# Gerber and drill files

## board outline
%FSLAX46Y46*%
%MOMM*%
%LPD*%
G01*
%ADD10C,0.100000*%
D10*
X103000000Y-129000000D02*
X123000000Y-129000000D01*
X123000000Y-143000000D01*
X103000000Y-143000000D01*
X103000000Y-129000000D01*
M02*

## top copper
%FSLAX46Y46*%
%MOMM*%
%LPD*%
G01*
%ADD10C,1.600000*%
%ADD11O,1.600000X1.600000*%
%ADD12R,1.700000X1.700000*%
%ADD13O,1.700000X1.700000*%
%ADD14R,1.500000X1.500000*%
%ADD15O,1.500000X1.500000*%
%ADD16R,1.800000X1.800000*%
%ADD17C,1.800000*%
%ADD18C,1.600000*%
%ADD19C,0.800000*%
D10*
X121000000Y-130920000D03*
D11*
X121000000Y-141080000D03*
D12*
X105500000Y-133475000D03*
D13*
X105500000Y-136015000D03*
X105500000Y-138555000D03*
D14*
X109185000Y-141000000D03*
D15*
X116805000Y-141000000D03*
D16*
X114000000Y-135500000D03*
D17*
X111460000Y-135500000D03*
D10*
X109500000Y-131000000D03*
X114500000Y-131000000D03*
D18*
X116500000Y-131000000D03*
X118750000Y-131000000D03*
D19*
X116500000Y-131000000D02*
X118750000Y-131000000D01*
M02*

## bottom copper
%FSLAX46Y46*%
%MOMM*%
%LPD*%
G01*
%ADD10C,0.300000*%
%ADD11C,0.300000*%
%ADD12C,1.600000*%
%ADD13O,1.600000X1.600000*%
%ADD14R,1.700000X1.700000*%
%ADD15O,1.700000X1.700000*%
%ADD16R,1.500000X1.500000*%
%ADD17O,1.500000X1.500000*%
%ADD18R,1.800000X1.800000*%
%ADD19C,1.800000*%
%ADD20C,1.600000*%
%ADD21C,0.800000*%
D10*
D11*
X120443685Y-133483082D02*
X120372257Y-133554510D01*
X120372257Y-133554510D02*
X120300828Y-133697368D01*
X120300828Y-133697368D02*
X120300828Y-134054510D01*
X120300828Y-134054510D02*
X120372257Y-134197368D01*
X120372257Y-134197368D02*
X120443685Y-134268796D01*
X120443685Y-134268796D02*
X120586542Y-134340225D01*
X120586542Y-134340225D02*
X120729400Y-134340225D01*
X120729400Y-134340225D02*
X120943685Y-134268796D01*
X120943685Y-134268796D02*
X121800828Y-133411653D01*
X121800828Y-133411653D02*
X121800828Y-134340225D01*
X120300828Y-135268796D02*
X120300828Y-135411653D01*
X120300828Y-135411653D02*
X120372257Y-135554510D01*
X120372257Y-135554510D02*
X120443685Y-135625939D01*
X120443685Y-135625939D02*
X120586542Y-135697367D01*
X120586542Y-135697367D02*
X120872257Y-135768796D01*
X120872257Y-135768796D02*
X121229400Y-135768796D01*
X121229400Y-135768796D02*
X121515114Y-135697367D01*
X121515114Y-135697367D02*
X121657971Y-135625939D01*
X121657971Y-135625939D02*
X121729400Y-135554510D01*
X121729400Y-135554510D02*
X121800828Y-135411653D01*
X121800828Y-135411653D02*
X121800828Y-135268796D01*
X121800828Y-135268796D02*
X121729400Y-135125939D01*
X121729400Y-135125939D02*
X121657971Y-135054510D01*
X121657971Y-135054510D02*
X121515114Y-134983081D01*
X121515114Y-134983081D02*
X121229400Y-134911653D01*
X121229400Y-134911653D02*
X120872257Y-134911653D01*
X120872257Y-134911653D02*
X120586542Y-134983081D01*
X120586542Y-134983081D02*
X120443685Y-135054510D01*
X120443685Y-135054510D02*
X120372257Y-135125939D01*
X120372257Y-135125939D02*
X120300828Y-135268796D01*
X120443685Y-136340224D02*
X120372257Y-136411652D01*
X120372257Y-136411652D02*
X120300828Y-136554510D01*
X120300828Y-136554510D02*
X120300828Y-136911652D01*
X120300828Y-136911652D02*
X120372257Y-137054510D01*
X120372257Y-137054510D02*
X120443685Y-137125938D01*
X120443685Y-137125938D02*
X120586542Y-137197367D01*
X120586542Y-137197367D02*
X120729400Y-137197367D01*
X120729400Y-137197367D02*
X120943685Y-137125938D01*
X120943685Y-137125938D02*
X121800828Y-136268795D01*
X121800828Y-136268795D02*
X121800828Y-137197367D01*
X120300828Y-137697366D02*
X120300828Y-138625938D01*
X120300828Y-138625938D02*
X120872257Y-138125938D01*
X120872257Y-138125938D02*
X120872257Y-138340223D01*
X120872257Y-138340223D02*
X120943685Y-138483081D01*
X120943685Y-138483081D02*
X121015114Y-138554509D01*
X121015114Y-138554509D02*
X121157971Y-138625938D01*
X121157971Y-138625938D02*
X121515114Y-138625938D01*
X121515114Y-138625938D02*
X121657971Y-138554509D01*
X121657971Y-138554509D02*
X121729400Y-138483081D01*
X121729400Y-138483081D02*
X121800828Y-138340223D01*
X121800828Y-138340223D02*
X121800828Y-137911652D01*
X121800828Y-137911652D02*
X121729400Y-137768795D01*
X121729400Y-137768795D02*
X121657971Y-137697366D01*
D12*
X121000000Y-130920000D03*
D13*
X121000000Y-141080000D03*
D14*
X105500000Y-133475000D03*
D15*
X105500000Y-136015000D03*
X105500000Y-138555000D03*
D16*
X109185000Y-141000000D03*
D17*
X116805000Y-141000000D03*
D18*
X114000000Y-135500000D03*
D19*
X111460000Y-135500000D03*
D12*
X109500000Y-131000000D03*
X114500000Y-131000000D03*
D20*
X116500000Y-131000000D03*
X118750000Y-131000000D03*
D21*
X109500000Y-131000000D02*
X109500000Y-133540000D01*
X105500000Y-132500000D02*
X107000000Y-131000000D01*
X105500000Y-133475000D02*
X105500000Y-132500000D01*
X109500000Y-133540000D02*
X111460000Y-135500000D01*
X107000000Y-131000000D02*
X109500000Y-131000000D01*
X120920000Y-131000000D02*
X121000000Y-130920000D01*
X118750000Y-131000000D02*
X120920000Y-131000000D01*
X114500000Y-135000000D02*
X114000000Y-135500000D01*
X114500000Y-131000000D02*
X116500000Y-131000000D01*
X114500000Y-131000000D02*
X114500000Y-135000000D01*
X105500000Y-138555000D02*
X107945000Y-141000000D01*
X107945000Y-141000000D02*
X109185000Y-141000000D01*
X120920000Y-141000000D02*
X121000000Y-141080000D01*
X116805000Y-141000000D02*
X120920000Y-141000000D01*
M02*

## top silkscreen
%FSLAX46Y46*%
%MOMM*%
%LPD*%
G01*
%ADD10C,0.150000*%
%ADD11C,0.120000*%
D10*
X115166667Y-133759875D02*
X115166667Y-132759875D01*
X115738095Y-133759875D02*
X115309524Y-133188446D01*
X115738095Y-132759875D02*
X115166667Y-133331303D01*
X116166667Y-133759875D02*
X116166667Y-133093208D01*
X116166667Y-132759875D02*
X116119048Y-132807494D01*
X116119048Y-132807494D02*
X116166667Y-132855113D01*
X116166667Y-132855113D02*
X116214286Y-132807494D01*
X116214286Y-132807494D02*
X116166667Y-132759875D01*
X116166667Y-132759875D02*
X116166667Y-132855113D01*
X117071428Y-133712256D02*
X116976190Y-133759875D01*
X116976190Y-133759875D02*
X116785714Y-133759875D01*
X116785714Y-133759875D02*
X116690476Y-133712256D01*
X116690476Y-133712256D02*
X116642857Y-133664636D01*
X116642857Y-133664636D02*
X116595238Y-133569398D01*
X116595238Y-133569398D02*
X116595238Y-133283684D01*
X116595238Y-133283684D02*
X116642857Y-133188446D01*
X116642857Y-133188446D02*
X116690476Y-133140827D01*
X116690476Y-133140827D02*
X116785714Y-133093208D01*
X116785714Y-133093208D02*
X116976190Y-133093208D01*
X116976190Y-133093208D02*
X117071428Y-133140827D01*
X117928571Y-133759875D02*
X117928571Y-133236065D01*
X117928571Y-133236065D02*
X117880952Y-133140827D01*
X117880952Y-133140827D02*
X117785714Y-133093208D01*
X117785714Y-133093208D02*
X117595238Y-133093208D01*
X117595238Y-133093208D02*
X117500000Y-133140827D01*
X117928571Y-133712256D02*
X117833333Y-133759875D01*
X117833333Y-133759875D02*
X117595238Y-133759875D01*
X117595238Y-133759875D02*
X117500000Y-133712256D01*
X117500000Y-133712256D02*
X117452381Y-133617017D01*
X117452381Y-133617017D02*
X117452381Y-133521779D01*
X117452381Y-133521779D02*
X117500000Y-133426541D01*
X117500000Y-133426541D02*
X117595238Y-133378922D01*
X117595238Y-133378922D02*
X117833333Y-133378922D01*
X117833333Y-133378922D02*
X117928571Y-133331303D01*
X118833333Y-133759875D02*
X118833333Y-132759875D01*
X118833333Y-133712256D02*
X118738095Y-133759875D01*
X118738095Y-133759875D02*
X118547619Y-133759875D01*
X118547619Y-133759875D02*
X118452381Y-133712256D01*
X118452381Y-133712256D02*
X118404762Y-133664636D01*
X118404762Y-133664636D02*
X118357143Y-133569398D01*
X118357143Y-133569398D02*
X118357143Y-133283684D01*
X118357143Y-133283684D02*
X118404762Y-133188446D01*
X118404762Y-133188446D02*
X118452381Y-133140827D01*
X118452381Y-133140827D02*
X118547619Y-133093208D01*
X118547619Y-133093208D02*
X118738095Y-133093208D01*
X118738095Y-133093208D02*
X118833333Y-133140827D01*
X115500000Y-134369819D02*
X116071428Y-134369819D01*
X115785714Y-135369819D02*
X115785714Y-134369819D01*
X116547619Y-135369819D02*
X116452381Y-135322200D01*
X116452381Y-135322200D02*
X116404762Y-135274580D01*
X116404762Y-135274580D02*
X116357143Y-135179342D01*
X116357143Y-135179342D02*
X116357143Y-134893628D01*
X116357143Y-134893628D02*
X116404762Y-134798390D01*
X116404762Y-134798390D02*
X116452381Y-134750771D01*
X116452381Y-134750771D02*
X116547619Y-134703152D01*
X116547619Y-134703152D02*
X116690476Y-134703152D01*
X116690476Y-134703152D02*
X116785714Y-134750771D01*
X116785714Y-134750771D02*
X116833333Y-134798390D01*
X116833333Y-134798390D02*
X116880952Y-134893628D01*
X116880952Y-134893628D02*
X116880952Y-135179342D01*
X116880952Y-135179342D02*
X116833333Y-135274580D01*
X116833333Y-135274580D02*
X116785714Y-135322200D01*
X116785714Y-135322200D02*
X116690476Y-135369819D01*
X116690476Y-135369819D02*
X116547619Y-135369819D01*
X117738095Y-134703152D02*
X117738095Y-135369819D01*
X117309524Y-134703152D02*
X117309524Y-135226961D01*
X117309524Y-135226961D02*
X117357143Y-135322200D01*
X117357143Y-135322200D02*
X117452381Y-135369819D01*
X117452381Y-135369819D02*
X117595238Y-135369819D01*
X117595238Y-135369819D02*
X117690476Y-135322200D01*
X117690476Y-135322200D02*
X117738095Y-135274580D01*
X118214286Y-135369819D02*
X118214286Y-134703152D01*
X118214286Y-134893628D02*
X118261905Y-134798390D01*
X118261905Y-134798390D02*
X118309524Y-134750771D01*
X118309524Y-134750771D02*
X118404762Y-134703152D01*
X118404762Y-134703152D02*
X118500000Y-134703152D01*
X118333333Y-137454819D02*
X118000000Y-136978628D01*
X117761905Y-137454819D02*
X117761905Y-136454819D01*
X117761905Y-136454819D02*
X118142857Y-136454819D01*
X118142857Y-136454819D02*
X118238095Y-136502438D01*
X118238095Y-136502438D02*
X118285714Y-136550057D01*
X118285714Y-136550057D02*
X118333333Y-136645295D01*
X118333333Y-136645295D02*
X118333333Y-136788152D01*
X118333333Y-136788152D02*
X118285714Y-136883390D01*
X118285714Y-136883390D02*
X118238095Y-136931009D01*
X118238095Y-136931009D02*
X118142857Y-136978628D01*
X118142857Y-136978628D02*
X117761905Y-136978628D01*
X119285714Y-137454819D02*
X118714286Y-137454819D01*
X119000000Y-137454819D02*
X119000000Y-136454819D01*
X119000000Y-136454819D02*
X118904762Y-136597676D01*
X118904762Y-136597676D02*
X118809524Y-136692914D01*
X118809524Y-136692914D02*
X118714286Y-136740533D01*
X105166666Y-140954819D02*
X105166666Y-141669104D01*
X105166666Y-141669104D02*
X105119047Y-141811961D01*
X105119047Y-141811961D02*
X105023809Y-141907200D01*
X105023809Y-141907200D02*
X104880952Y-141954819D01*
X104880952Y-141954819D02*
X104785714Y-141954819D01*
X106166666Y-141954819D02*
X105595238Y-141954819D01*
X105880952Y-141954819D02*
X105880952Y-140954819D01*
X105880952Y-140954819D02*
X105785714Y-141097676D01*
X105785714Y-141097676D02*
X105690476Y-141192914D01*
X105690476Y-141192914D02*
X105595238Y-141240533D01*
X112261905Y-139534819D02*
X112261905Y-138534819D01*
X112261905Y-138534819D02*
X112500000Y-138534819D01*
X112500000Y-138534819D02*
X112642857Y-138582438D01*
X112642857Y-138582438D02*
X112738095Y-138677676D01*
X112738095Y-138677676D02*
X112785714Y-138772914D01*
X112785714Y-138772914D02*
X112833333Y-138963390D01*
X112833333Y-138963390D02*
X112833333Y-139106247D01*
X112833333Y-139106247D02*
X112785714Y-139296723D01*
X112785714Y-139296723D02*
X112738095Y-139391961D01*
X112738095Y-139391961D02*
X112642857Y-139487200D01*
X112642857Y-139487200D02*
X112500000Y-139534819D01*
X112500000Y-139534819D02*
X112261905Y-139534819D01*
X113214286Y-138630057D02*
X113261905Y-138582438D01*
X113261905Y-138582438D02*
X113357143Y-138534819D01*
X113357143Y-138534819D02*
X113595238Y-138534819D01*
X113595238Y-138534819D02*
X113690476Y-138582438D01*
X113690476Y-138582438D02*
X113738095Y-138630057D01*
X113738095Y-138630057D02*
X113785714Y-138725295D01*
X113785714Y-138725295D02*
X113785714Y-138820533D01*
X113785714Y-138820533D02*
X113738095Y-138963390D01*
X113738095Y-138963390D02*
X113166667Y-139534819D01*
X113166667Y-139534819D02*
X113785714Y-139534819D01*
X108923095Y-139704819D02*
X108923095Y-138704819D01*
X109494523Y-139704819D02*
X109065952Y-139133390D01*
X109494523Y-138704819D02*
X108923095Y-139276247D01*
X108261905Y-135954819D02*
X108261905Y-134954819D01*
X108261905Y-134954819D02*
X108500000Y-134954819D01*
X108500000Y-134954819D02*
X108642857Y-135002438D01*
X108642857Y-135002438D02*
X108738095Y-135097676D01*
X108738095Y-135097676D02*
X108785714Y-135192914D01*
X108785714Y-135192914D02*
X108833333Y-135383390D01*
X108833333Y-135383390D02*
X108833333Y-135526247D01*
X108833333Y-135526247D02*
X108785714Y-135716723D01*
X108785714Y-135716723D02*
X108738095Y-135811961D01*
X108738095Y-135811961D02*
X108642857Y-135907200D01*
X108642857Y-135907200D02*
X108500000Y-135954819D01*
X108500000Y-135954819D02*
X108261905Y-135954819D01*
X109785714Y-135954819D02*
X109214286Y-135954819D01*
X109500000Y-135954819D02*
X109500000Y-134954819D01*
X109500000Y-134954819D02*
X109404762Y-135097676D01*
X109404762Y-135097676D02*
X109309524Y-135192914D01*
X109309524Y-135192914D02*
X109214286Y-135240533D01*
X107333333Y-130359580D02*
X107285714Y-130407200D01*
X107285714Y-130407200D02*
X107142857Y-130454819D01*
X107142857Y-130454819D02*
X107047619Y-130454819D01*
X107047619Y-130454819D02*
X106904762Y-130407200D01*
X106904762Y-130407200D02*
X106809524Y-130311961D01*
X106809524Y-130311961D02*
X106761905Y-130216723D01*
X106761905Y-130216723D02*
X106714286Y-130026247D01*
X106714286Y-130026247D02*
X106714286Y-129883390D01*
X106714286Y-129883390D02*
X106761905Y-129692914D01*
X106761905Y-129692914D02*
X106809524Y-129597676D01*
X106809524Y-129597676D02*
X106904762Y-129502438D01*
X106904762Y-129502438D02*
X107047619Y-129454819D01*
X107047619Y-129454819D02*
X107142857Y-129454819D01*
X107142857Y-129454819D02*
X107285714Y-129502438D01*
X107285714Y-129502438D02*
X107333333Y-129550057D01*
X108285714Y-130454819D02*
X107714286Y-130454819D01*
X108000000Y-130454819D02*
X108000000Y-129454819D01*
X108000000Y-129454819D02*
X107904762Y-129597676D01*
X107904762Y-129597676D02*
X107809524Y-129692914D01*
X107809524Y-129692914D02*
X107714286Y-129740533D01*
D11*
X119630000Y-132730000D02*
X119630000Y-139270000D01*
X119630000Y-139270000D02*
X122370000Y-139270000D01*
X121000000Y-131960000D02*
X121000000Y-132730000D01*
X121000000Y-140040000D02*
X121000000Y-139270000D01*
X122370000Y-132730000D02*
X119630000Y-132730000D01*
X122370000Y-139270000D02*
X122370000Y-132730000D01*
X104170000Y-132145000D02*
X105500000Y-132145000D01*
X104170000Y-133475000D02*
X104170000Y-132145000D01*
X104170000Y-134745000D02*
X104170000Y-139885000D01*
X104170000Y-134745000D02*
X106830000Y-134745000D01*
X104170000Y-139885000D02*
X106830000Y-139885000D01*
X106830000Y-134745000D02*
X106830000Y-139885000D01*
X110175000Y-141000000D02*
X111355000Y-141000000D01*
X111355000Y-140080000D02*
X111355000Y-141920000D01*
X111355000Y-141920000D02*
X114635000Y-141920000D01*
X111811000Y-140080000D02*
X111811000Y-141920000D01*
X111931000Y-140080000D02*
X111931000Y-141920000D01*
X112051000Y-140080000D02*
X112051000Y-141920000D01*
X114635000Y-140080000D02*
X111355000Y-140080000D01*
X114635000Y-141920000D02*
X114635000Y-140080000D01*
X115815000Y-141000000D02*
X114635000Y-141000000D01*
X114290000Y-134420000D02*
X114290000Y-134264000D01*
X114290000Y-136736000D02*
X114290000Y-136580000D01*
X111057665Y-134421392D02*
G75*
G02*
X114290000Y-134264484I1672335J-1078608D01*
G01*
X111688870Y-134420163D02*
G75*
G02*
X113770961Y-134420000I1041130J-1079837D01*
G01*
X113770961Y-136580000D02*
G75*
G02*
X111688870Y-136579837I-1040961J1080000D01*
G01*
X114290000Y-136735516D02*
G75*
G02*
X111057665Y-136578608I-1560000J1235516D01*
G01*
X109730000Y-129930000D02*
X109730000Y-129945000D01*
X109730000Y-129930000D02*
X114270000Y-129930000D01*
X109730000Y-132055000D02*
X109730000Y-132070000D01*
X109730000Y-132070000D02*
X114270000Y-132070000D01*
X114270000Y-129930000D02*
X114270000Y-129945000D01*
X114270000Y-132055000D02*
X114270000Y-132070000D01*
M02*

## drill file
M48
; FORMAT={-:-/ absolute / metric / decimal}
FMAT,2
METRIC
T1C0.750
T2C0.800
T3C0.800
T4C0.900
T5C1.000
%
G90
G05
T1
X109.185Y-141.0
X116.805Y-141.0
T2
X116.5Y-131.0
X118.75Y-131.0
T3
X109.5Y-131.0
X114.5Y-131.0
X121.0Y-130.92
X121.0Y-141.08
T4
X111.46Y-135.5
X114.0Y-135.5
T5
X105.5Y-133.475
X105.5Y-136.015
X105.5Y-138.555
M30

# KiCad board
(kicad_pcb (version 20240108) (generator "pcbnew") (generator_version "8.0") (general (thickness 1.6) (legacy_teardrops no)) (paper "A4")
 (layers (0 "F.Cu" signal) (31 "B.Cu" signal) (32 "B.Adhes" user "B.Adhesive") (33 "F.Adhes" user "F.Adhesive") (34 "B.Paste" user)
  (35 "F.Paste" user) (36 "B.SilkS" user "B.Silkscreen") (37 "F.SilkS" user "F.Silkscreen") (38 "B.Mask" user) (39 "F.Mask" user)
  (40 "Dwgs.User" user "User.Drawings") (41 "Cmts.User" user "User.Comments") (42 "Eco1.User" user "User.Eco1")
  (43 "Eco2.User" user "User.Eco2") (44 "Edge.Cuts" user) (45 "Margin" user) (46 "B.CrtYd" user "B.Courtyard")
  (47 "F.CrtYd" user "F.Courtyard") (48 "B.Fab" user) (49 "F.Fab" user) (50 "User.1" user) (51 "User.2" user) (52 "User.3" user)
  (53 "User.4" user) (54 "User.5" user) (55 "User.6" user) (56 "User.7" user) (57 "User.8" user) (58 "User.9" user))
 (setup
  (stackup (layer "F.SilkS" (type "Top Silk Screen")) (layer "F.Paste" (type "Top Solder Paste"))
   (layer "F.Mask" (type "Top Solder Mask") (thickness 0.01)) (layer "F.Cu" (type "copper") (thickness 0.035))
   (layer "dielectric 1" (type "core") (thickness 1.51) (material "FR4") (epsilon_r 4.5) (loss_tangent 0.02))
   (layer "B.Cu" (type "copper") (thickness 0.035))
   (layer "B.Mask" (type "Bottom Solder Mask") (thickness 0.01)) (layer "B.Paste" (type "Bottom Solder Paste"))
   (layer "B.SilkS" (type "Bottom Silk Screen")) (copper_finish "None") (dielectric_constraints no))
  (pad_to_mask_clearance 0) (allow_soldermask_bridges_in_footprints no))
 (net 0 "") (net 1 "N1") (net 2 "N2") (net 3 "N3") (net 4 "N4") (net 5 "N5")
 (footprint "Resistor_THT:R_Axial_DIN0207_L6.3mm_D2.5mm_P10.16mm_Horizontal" (layer "F.Cu") (at 121 130.92 -90)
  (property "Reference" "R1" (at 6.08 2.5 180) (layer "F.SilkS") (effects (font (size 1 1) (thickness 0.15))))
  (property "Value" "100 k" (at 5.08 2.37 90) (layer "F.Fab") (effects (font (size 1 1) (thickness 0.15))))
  (fp_line (start 1.81 1.37) (end 8.35 1.37) (stroke (width 0.12) (type solid)) (layer "F.SilkS"))
  (fp_line (start 8.35 1.37) (end 8.35 -1.37) (stroke (width 0.12) (type solid)) (layer "F.SilkS"))
  (fp_line (start 1.04 0) (end 1.81 0) (stroke (width 0.12) (type solid)) (layer "F.SilkS"))
  (fp_line (start 9.12 0) (end 8.35 0) (stroke (width 0.12) (type solid)) (layer "F.SilkS"))
  (fp_line (start 1.81 -1.37) (end 1.81 1.37) (stroke (width 0.12) (type solid)) (layer "F.SilkS"))
  (fp_line (start 8.35 -1.37) (end 1.81 -1.37) (stroke (width 0.12) (type solid)) (layer "F.SilkS"))
  (pad "1" thru_hole circle (at 0 0 270) (size 1.6 1.6) (drill 0.8) (layers "*.Cu" "*.Mask") (remove_unused_layers no) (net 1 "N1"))
  (pad "2" thru_hole oval (at 10.16 0 270) (size 1.6 1.6) (drill 0.8) (layers "*.Cu" "*.Mask") (remove_unused_layers no) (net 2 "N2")))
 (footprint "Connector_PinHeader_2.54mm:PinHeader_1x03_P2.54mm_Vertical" (layer "F.Cu") (at 105.5 133.475)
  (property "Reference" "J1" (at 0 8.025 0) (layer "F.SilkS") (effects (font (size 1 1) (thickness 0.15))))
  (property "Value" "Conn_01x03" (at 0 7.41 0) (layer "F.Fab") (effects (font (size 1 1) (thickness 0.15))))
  (fp_line (start -1.33 -1.33) (end 0 -1.33) (stroke (width 0.12) (type solid)) (layer "F.SilkS"))
  (fp_line (start -1.33 0) (end -1.33 -1.33) (stroke (width 0.12) (type solid)) (layer "F.SilkS"))
  (fp_line (start -1.33 1.27) (end -1.33 6.41) (stroke (width 0.12) (type solid)) (layer "F.SilkS"))
  (fp_line (start -1.33 1.27) (end 1.33 1.27) (stroke (width 0.12) (type solid)) (layer "F.SilkS"))
  (fp_line (start -1.33 6.41) (end 1.33 6.41) (stroke (width 0.12) (type solid)) (layer "F.SilkS"))
  (fp_line (start 1.33 1.27) (end 1.33 6.41) (stroke (width 0.12) (type solid)) (layer "F.SilkS"))
  (pad "1" thru_hole rect (at 0 0) (size 1.7 1.7) (drill 1) (layers "*.Cu" "*.Mask") (remove_unused_layers no) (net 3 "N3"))
  (pad "2" thru_hole oval (at 0 2.54) (size 1.7 1.7) (drill 1) (layers "*.Cu" "*.Mask") (remove_unused_layers no) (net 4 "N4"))
  (pad "3" thru_hole oval (at 0 5.08) (size 1.7 1.7) (drill 1) (layers "*.Cu" "*.Mask") (remove_unused_layers no) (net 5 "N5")))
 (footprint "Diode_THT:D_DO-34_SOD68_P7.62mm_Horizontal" (layer "F.Cu") (at 109.185 141)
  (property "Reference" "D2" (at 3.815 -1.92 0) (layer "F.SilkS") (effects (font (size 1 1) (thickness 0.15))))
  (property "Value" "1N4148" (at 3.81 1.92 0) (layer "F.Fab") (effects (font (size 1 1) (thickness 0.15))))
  (fp_line (start 0.99 0) (end 2.17 0) (stroke (width 0.12) (type solid)) (layer "F.SilkS"))
  (fp_line (start 2.17 -0.92) (end 2.17 0.92) (stroke (width 0.12) (type solid)) (layer "F.SilkS"))
  (fp_line (start 2.17 0.92) (end 5.45 0.92) (stroke (width 0.12) (type solid)) (layer "F.SilkS"))
  (fp_line (start 2.626 -0.92) (end 2.626 0.92) (stroke (width 0.12) (type solid)) (layer "F.SilkS"))
  (fp_line (start 2.746 -0.92) (end 2.746 0.92) (stroke (width 0.12) (type solid)) (layer "F.SilkS"))
  (fp_line (start 2.866 -0.92) (end 2.866 0.92) (stroke (width 0.12) (type solid)) (layer "F.SilkS"))
  (fp_line (start 5.45 -0.92) (end 2.17 -0.92) (stroke (width 0.12) (type solid)) (layer "F.SilkS"))
  (fp_line (start 5.45 0.92) (end 5.45 -0.92) (stroke (width 0.12) (type solid)) (layer "F.SilkS"))
  (fp_line (start 6.63 0) (end 5.45 0) (stroke (width 0.12) (type solid)) (layer "F.SilkS"))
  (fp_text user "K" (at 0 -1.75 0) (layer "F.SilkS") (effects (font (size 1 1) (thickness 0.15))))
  (pad "1" thru_hole rect (at 0 0) (size 1.5 1.5) (drill 0.75) (layers "*.Cu" "*.Mask") (remove_unused_layers no) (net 5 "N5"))
  (pad "2" thru_hole oval (at 7.62 0) (size 1.5 1.5) (drill 0.75) (layers "*.Cu" "*.Mask") (remove_unused_layers no) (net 2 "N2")))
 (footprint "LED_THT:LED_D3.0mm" (layer "F.Cu") (at 114 135.5 180)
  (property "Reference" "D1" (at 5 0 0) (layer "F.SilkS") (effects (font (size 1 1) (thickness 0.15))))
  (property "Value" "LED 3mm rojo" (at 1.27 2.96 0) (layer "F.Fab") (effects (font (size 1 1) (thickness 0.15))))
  (fp_line (start -0.29 1.08) (end -0.29 1.236) (stroke (width 0.12) (type solid)) (layer "F.SilkS"))
  (fp_line (start -0.29 -1.236) (end -0.29 -1.08) (stroke (width 0.12) (type solid)) (layer "F.SilkS"))
  (fp_arc (start 2.942335 1.078608) (mid 1.366487 1.987659) (end -0.29 1.235516) (stroke (width 0.12) (type solid)) (layer "F.SilkS"))
  (fp_arc (start 2.31113 1.079837) (mid 1.270117 1.5) (end 0.229039 1.08) (stroke (width 0.12) (type solid)) (layer "F.SilkS"))
  (fp_arc (start 0.229039 -1.08) (mid 1.270117 -1.5) (end 2.31113 -1.079837) (stroke (width 0.12) (type solid)) (layer "F.SilkS"))
  (fp_arc (start -0.29 -1.235516) (mid 1.366487 -1.987659) (end 2.942335 -1.078608) (stroke (width 0.12) (type solid)) (layer "F.SilkS"))
  (pad "1" thru_hole rect (at 0 0 180) (size 1.8 1.8) (drill 0.9) (layers "*.Cu" "*.Mask") (remove_unused_layers no) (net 1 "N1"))
  (pad "2" thru_hole circle (at 2.54 0 180) (size 1.8 1.8) (drill 0.9) (layers "*.Cu" "*.Mask") (remove_unused_layers no) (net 3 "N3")))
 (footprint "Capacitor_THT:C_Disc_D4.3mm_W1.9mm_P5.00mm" (layer "F.Cu") (at 109.5 131)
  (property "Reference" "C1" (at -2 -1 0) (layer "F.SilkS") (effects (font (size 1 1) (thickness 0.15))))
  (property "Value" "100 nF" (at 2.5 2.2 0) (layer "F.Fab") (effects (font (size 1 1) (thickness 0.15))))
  (fp_line (start 0.23 -1.07) (end 0.23 -1.055) (stroke (width 0.12) (type solid)) (layer "F.SilkS"))
  (fp_line (start 0.23 -1.07) (end 4.77 -1.07) (stroke (width 0.12) (type solid)) (layer "F.SilkS"))
  (fp_line (start 0.23 1.055) (end 0.23 1.07) (stroke (width 0.12) (type solid)) (layer "F.SilkS"))
  (fp_line (start 0.23 1.07) (end 4.77 1.07) (stroke (width 0.12) (type solid)) (layer "F.SilkS"))
  (fp_line (start 4.77 -1.07) (end 4.77 -1.055) (stroke (width 0.12) (type solid)) (layer "F.SilkS"))
  (fp_line (start 4.77 1.055) (end 4.77 1.07) (stroke (width 0.12) (type solid)) (layer "F.SilkS"))
  (pad "1" thru_hole circle (at 0 0) (size 1.6 1.6) (drill 0.8) (layers "*.Cu" "*.Mask") (remove_unused_layers no) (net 3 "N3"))
  (pad "2" thru_hole circle (at 5 0) (size 1.6 1.6) (drill 0.8) (layers "*.Cu" "*.Mask") (remove_unused_layers no) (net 1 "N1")))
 (gr_rect (start 103 129) (end 123 143) (stroke (width 0.1) (type default)) (fill none) (layer "Edge.Cuts"))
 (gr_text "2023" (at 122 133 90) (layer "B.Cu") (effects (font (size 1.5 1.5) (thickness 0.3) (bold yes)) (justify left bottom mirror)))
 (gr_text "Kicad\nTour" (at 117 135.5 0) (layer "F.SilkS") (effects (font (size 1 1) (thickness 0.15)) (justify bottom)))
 (segment (start 109.5 131) (end 109.5 133.54) (width 0.8) (layer "B.Cu") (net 3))
 (segment (start 105.5 132.5) (end 107 131) (width 0.8) (layer "B.Cu") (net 3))
 (segment (start 105.5 133.475) (end 105.5 132.5) (width 0.8) (layer "B.Cu") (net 3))
 (segment (start 109.5 133.54) (end 111.46 135.5) (width 0.8) (layer "B.Cu") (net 3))
 (segment (start 107 131) (end 109.5 131) (width 0.8) (layer "B.Cu") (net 3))
 (segment (start 116.5 131) (end 118.75 131) (width 0.8) (layer "F.Cu") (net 1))
 (via (at 116.5 131) (size 1.6) (drill 0.8) (layers "F.Cu" "B.Cu") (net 1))
 (via (at 118.75 131) (size 1.6) (drill 0.8) (layers "F.Cu" "B.Cu") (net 1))
 (segment (start 120.92 131) (end 121 130.92) (width 0.8) (layer "B.Cu") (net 1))
 (segment (start 118.75 131) (end 120.92 131) (width 0.8) (layer "B.Cu") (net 1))
 (segment (start 114.5 135) (end 114 135.5) (width 0.8) (layer "B.Cu") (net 1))
 (segment (start 114.5 131) (end 116.5 131) (width 0.8) (layer "B.Cu") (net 1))
 (segment (start 114.5 131) (end 114.5 135) (width 0.8) (layer "B.Cu") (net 1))
 (segment (start 105.5 138.555) (end 107.945 141) (width 0.8) (layer "B.Cu") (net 5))
 (segment (start 107.945 141) (end 109.185 141) (width 0.8) (layer "B.Cu") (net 5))
 (segment (start 120.92 141) (end 121 141.08) (width 0.8) (layer "B.Cu") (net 2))
 (segment (start 116.805 141) (end 120.92 141) (width 0.8) (layer "B.Cu") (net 2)))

